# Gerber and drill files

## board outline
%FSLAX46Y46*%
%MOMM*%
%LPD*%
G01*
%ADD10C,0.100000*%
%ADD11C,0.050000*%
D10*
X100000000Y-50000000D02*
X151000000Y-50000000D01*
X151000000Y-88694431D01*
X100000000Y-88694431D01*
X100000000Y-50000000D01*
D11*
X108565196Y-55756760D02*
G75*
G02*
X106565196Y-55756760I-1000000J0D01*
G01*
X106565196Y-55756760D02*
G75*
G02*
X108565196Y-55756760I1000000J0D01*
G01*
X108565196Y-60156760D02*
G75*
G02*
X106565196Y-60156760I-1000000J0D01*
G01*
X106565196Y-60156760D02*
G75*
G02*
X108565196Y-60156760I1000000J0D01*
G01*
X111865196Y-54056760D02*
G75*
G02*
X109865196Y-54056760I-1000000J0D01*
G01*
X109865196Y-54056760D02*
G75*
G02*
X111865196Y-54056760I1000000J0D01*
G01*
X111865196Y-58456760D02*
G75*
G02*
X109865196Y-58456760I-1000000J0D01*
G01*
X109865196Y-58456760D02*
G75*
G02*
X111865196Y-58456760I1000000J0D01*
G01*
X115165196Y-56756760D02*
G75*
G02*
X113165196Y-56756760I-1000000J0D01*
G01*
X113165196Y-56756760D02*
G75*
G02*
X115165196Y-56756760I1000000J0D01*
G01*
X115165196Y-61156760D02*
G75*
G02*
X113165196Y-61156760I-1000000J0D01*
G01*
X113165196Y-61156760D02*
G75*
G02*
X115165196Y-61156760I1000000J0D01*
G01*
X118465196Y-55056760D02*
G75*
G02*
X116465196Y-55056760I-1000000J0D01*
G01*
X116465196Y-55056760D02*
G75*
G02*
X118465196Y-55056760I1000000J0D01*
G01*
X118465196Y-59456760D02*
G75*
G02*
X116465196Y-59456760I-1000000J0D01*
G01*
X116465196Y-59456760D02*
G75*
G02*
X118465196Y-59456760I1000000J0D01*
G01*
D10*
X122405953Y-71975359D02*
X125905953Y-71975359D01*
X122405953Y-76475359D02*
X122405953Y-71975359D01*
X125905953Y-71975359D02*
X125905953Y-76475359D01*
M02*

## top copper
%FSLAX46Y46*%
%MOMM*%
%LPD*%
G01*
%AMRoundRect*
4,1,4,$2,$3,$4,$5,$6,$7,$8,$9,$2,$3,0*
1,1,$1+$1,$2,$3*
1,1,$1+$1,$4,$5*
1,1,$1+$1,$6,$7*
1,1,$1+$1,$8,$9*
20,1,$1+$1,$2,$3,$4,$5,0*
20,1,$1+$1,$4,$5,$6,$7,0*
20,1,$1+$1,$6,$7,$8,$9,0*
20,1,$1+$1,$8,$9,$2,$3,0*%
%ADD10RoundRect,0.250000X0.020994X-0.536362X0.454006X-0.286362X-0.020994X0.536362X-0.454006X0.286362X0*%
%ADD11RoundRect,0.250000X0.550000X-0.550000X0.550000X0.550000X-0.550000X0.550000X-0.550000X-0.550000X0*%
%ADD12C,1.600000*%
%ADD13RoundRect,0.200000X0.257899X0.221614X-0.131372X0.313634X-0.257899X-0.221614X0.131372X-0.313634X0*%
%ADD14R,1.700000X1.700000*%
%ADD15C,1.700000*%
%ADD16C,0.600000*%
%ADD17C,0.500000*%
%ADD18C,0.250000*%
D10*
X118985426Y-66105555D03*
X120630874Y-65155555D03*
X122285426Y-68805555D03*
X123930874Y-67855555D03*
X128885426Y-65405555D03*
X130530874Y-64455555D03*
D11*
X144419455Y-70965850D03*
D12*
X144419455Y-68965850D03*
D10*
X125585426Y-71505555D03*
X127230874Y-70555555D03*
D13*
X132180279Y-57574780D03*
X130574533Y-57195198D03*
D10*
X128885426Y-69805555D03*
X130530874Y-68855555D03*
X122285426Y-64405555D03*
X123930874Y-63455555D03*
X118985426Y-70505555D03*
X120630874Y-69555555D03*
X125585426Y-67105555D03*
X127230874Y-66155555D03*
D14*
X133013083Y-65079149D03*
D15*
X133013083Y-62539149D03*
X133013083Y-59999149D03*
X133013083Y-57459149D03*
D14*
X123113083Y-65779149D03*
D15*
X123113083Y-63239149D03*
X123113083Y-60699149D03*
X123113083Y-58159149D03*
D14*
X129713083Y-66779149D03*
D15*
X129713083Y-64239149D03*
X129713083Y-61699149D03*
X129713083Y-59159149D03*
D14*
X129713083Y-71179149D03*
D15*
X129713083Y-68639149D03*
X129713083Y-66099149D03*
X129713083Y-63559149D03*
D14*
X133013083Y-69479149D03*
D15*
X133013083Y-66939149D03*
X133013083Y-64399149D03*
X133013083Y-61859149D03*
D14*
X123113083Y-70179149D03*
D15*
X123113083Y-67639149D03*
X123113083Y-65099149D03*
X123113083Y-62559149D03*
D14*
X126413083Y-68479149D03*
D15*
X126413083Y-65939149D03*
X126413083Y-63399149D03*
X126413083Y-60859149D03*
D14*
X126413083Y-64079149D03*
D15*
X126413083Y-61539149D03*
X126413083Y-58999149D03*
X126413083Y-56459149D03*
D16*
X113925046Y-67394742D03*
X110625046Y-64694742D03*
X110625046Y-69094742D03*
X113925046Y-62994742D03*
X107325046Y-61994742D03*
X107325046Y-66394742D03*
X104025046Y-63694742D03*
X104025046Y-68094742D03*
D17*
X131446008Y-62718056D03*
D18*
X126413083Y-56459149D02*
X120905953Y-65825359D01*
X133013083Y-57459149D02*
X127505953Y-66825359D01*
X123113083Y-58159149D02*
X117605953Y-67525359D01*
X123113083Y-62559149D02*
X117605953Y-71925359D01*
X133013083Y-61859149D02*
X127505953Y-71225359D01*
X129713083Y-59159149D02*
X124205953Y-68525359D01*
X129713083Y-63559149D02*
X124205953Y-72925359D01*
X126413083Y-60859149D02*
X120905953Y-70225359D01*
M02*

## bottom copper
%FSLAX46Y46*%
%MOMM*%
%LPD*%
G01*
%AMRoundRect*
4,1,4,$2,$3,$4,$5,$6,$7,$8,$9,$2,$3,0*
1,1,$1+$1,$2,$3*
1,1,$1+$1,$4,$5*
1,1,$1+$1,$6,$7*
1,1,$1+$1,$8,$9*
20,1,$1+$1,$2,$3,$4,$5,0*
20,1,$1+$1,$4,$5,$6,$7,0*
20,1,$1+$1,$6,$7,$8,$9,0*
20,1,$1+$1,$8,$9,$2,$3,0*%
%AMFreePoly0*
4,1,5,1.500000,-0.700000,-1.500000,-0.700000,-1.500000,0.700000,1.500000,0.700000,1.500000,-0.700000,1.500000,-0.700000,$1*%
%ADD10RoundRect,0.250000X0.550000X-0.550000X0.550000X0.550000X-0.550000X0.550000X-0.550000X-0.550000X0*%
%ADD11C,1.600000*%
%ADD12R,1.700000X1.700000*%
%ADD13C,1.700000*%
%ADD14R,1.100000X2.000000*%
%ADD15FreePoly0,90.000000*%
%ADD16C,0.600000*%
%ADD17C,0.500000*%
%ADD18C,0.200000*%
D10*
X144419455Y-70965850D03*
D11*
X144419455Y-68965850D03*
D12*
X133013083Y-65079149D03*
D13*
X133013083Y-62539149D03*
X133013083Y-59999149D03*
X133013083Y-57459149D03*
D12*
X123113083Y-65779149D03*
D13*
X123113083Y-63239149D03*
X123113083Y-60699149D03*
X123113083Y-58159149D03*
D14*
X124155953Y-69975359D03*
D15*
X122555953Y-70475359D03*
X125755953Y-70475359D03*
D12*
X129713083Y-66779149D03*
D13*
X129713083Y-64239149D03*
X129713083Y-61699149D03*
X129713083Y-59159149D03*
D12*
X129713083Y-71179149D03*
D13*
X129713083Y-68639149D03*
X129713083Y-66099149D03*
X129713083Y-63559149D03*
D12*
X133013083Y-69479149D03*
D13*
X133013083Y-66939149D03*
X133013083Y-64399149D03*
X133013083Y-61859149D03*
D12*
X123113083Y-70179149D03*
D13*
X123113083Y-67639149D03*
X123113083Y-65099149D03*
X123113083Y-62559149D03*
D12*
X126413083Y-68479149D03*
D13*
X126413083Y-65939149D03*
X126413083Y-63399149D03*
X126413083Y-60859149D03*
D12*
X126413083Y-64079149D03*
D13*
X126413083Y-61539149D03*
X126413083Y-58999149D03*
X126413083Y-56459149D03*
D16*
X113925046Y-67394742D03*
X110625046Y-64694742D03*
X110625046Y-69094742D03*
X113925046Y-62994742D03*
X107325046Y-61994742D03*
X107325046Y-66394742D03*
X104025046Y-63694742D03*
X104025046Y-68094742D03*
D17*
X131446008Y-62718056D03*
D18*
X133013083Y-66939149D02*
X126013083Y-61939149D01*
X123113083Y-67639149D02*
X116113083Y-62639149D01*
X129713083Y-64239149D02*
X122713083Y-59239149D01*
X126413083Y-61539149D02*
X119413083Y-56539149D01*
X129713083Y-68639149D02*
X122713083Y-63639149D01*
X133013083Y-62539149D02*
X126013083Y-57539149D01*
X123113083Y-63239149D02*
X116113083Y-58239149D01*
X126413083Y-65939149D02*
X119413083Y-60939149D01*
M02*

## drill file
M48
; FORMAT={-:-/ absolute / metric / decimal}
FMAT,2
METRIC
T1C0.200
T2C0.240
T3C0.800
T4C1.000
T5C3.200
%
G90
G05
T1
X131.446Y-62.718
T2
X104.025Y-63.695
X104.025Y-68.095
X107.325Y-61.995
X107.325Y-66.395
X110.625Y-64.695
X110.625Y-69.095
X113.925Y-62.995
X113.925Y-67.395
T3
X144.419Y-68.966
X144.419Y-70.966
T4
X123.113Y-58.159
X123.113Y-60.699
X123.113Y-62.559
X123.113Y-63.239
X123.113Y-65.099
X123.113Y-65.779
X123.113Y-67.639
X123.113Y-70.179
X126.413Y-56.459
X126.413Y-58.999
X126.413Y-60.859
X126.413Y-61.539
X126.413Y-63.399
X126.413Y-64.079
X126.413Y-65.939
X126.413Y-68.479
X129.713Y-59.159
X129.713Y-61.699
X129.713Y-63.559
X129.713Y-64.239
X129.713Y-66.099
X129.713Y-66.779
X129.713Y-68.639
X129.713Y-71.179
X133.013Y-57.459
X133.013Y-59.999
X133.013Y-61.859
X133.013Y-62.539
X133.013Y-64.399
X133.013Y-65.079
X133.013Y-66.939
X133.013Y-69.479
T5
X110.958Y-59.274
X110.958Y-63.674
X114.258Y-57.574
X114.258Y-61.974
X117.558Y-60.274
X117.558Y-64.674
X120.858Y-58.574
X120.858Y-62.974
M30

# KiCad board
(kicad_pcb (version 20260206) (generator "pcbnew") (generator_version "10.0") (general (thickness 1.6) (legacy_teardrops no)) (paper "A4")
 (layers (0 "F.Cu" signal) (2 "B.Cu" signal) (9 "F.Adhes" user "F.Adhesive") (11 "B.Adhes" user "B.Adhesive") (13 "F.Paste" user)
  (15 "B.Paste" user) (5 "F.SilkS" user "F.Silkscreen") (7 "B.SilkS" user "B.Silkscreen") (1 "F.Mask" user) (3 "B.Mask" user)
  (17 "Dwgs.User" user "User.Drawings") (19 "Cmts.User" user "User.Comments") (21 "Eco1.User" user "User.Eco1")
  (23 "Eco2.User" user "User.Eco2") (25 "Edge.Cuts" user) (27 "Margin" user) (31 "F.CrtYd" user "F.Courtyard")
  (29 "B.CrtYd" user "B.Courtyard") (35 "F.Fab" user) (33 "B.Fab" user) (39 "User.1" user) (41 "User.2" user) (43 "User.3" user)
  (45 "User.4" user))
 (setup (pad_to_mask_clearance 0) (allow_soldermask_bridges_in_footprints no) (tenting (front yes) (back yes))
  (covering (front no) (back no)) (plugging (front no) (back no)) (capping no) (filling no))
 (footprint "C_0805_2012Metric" (layer "F.Cu") (at 119.80815 65.630555 30)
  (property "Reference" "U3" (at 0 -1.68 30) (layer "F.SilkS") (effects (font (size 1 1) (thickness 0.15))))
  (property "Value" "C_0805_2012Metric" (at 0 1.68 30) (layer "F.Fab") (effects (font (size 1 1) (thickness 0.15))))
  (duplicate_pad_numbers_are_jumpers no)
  (pad "1" smd roundrect (at -0.95 0 30) (size 1 1.45) (layers "F.Cu" "F.Mask" "F.Paste") (roundrect_rratio 0.25) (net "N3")
   (clearance 0.35))
  (pad "2" smd roundrect (at 0.95 0 30) (size 1 1.45) (layers "F.Cu" "F.Mask" "F.Paste") (roundrect_rratio 0.25)))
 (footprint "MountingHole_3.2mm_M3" (layer "F.Cu") (at 117.558484 64.674067 45)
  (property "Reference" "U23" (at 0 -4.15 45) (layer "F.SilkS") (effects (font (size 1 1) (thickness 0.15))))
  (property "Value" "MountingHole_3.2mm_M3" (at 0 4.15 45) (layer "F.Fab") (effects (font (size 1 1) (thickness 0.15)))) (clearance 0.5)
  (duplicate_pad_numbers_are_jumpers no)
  (pad "" np_thru_hole circle (at 0 0 45) (size 3.2 3.2) (drill 3.2) (layers "*.Cu" "*.Mask")))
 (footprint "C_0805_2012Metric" (layer "F.Cu") (at 123.10815 68.330555 30)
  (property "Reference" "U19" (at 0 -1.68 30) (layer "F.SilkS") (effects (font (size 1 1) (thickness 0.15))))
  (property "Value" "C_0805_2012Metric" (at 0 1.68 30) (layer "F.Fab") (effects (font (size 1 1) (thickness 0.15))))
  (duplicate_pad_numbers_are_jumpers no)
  (pad "1" smd roundrect (at -0.95 0 30) (size 1 1.45) (layers "F.Cu" "F.Mask" "F.Paste") (roundrect_rratio 0.25) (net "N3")
   (clearance 0.35))
  (pad "2" smd roundrect (at 0.95 0 30) (size 1 1.45) (layers "F.Cu" "F.Mask" "F.Paste") (roundrect_rratio 0.25)))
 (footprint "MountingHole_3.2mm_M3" (layer "F.Cu") (at 114.258484 57.574067 45)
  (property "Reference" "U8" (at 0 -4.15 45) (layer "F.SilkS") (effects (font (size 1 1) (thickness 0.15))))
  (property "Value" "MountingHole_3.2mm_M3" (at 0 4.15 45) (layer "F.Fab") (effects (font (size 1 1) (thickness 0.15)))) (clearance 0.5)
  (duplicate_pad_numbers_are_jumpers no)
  (pad "" np_thru_hole circle (at 0 0 45) (size 3.2 3.2) (drill 3.2) (layers "*.Cu" "*.Mask")))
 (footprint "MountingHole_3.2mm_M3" (layer "F.Cu") (at 114.258484 61.974067 45)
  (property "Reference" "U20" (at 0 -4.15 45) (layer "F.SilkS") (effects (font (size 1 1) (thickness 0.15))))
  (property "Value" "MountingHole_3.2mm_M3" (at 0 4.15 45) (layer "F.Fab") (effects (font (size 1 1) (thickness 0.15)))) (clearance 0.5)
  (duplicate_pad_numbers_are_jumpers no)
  (pad "" np_thru_hole circle (at 0 0 45) (size 3.2 3.2) (drill 3.2) (layers "*.Cu" "*.Mask")))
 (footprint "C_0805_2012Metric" (layer "F.Cu") (at 129.70815 64.930555 30)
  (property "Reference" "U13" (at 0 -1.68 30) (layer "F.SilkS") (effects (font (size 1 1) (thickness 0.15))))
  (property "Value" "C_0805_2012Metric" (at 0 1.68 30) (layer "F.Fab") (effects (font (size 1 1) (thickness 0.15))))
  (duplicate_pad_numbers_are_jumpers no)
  (pad "1" smd roundrect (at -0.95 0 30) (size 1 1.45) (layers "F.Cu" "F.Mask" "F.Paste") (roundrect_rratio 0.25) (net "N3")
   (clearance 0.35))
  (pad "2" smd roundrect (at 0.95 0 30) (size 1 1.45) (layers "F.Cu" "F.Mask" "F.Paste") (roundrect_rratio 0.25)))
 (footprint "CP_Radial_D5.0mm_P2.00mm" (layer "F.Cu") (at 144.419455 70.96585 90)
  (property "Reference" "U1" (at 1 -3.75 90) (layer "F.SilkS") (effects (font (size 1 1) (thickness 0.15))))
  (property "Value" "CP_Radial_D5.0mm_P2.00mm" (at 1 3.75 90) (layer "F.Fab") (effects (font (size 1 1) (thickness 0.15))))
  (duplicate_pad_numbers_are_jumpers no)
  (pad "1" thru_hole roundrect (at 0 0 90) (size 1.6 1.6) (drill 0.8) (layers "*.Cu" "*.Mask") (remove_unused_layers no)
   (roundrect_rratio 0.15625) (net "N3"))
  (pad "2" thru_hole circle (at 2 0 90) (size 1.6 1.6) (drill 0.8) (layers "*.Cu" "*.Mask") (remove_unused_layers no) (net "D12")))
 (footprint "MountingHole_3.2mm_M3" (layer "F.Cu") (at 117.558484 60.274067 45)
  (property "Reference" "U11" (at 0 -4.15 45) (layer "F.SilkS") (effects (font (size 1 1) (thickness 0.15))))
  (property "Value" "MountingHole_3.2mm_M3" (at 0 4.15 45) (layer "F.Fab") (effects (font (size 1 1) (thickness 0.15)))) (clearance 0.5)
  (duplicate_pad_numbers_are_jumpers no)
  (pad "" np_thru_hole circle (at 0 0 45) (size 3.2 3.2) (drill 3.2) (layers "*.Cu" "*.Mask")))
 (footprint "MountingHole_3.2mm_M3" (layer "F.Cu") (at 110.958484 59.274067 45)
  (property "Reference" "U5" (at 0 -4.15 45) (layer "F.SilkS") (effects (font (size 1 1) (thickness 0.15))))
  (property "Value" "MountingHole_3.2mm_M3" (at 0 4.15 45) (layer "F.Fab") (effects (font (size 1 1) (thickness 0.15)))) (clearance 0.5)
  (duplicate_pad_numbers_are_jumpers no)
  (pad "" np_thru_hole circle (at 0 0 45) (size 3.2 3.2) (drill 3.2) (layers "*.Cu" "*.Mask")))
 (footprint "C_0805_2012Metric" (layer "F.Cu") (at 126.40815 71.030555 30)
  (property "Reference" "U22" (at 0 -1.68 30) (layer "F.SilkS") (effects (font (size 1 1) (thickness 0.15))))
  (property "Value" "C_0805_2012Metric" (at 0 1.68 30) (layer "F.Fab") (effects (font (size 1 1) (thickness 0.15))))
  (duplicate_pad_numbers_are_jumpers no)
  (pad "1" smd roundrect (at -0.95 0 30) (size 1 1.45) (layers "F.Cu" "F.Mask" "F.Paste") (roundrect_rratio 0.25) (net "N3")
   (clearance 0.35))
  (pad "2" smd roundrect (at 0.95 0 30) (size 1 1.45) (layers "F.Cu" "F.Mask" "F.Paste") (roundrect_rratio 0.25)))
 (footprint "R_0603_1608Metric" (layer "F.Cu") (at 131.377406 57.384989 166.7)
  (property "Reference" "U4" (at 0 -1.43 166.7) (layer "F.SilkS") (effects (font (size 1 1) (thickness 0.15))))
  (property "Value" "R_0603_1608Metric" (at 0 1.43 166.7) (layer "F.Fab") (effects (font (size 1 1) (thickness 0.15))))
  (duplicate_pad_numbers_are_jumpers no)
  (pad "1" smd roundrect (at -0.825 0 166.7) (size 0.8 0.95) (layers "F.Cu" "F.Mask" "F.Paste") (roundrect_rratio 0.25) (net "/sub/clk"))
  (pad "2" smd roundrect (at 0.825 0 166.7) (size 0.8 0.95) (layers "F.Cu" "F.Mask" "F.Paste") (roundrect_rratio 0.25) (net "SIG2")))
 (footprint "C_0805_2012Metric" (layer "F.Cu") (at 129.70815 69.330555 30)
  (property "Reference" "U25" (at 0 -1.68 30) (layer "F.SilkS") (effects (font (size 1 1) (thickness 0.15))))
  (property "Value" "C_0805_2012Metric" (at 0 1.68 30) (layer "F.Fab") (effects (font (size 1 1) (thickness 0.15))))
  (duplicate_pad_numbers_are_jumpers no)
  (pad "1" smd roundrect (at -0.95 0 30) (size 1 1.45) (layers "F.Cu" "F.Mask" "F.Paste") (roundrect_rratio 0.25) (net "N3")
   (clearance 0.35))
  (pad "2" smd roundrect (at 0.95 0 30) (size 1 1.45) (layers "F.Cu" "F.Mask" "F.Paste") (roundrect_rratio 0.25)))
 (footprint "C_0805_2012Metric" (layer "F.Cu") (at 123.10815 63.930555 30)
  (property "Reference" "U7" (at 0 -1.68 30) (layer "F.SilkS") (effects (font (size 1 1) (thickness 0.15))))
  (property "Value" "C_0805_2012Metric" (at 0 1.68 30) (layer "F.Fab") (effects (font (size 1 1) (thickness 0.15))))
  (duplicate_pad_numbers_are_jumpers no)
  (pad "1" smd roundrect (at -0.95 0 30) (size 1 1.45) (layers "F.Cu" "F.Mask" "F.Paste") (roundrect_rratio 0.25) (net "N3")
   (clearance 0.35))
  (pad "2" smd roundrect (at 0.95 0 30) (size 1 1.45) (layers "F.Cu" "F.Mask" "F.Paste") (roundrect_rratio 0.25)))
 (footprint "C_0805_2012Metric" (layer "F.Cu") (at 119.80815 70.030555 30)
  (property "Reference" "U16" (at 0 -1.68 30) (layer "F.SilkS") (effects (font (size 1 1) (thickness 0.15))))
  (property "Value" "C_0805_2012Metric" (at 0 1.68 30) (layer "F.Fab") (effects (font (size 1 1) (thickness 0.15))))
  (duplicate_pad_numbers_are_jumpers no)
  (pad "1" smd roundrect (at -0.95 0 30) (size 1 1.45) (layers "F.Cu" "F.Mask" "F.Paste") (roundrect_rratio 0.25) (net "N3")
   (clearance 0.35))
  (pad "2" smd roundrect (at 0.95 0 30) (size 1 1.45) (layers "F.Cu" "F.Mask" "F.Paste") (roundrect_rratio 0.25)))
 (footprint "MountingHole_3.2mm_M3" (layer "F.Cu") (at 110.958484 63.674067 45)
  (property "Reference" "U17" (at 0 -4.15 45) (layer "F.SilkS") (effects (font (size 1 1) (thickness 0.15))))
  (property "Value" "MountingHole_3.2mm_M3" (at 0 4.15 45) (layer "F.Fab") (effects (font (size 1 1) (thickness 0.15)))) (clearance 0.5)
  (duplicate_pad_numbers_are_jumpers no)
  (pad "" np_thru_hole circle (at 0 0 45) (size 3.2 3.2) (drill 3.2) (layers "*.Cu" "*.Mask")))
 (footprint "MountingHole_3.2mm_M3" (layer "F.Cu") (at 120.858484 58.574067 45)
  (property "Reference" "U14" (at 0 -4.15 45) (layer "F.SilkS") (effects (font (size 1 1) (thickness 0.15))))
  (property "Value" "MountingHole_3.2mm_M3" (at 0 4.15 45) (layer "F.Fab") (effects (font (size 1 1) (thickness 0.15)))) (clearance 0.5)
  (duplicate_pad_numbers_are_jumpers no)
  (pad "" np_thru_hole circle (at 0 0 45) (size 3.2 3.2) (drill 3.2) (layers "*.Cu" "*.Mask")))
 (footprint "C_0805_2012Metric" (layer "F.Cu") (at 126.40815 66.630555 30)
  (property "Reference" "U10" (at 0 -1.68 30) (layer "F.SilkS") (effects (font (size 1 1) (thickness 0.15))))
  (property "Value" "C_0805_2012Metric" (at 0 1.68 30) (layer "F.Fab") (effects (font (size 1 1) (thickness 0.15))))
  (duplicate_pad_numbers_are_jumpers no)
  (pad "1" smd roundrect (at -0.95 0 30) (size 1 1.45) (layers "F.Cu" "F.Mask" "F.Paste") (roundrect_rratio 0.25) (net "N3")
   (clearance 0.35))
  (pad "2" smd roundrect (at 0.95 0 30) (size 1 1.45) (layers "F.Cu" "F.Mask" "F.Paste") (roundrect_rratio 0.25)))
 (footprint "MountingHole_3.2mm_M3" (layer "F.Cu") (at 120.858484 62.974067 45)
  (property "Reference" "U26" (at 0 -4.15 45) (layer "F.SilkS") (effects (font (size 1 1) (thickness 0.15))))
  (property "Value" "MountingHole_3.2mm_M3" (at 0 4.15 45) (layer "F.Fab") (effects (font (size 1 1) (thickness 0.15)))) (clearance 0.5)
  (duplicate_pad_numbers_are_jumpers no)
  (pad "" np_thru_hole circle (at 0 0 45) (size 3.2 3.2) (drill 3.2) (layers "*.Cu" "*.Mask")))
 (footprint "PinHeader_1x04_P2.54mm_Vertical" (layer "B.Cu") (at 133.013083 65.079149)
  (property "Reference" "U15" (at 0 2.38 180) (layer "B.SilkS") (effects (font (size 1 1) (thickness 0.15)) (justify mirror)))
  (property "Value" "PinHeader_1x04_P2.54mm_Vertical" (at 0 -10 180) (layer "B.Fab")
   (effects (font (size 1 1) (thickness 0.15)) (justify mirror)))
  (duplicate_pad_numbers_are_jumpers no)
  (pad "1" thru_hole rect (at 0 0) (size 1.7 1.7) (drill 1) (layers "*.Cu" "*.Mask") (remove_unused_layers no) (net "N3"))
  (pad "2" thru_hole circle (at 0 -2.54) (size 1.7 1.7) (drill 1) (layers "*.Cu" "*.Mask") (remove_unused_layers no) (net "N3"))
  (pad "3" thru_hole circle (at 0 -5.08) (size 1.7 1.7) (drill 1) (layers "*.Cu" "*.Mask") (remove_unused_layers no) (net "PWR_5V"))
  (pad "4" thru_hole circle (at 0 -7.62) (size 1.7 1.7) (drill 1) (layers "*.Cu" "*.Mask") (remove_unused_layers no)))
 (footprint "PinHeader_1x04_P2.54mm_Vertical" (layer "B.Cu") (at 123.113083 65.779149)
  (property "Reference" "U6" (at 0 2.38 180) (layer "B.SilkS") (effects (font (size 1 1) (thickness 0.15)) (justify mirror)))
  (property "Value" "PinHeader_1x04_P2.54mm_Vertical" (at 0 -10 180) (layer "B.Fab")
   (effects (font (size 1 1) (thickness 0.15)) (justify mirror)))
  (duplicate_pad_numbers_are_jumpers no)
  (pad "1" thru_hole rect (at 0 0) (size 1.7 1.7) (drill 1) (layers "*.Cu" "*.Mask") (remove_unused_layers no) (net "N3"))
  (pad "2" thru_hole circle (at 0 -2.54) (size 1.7 1.7) (drill 1) (layers "*.Cu" "*.Mask") (remove_unused_layers no) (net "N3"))
  (pad "3" thru_hole circle (at 0 -5.08) (size 1.7 1.7) (drill 1) (layers "*.Cu" "*.Mask") (remove_unused_layers no) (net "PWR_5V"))
  (pad "4" thru_hole circle (at 0 -7.62) (size 1.7 1.7) (drill 1) (layers "*.Cu" "*.Mask") (remove_unused_layers no)))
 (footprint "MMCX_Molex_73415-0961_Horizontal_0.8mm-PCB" (layer "B.Cu") (at 124.155953 72.725359 90)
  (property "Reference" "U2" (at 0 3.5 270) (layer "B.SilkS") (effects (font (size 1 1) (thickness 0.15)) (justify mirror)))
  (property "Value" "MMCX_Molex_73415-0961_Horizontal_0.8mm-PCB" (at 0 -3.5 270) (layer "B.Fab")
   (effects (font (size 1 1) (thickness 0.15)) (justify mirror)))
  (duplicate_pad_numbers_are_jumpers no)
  (fp_line (start 0.75 -1.75) (end 0.75 1.75) (stroke (width 0.1) (type solid)) (layer "Edge.Cuts"))
  (fp_line (start -3.75 -1.75) (end 0.75 -1.75) (stroke (width 0.1) (type solid)) (layer "Edge.Cuts"))
  (fp_line (start 0.75 1.75) (end -3.75 1.75) (stroke (width 0.1) (type solid)) (layer "Edge.Cuts"))
  (pad "1" smd rect (at 2.75 0 90) (size 2 1.1) (layers "B.Cu" "B.Mask" "B.Paste") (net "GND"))
  (pad "2" smd custom (at 2.25 -1.6 90) (size 3 1.4) (layers "B.Cu" "B.Mask" "B.Paste") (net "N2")
   (options (clearance outline) (anchor rect)) (primitives))
  (pad "2" smd custom (at 2.25 1.6 90) (size 3 1.4) (layers "B.Cu" "B.Mask" "B.Paste") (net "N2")
   (options (clearance outline) (anchor rect)) (primitives)))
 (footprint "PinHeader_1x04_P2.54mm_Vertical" (layer "B.Cu") (at 129.713083 66.779149)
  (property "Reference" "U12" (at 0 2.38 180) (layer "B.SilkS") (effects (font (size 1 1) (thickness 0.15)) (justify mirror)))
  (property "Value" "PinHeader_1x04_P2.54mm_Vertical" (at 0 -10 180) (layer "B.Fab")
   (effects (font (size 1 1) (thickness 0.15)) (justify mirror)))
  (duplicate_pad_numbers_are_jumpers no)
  (pad "1" thru_hole rect (at 0 0) (size 1.7 1.7) (drill 1) (layers "*.Cu" "*.Mask") (remove_unused_layers no) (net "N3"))
  (pad "2" thru_hole circle (at 0 -2.54) (size 1.7 1.7) (drill 1) (layers "*.Cu" "*.Mask") (remove_unused_layers no) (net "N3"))
  (pad "3" thru_hole circle (at 0 -5.08) (size 1.7 1.7) (drill 1) (layers "*.Cu" "*.Mask") (remove_unused_layers no) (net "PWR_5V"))
  (pad "4" thru_hole circle (at 0 -7.62) (size 1.7 1.7) (drill 1) (layers "*.Cu" "*.Mask") (remove_unused_layers no)))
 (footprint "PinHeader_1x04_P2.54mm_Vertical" (layer "B.Cu") (at 129.713083 71.179149)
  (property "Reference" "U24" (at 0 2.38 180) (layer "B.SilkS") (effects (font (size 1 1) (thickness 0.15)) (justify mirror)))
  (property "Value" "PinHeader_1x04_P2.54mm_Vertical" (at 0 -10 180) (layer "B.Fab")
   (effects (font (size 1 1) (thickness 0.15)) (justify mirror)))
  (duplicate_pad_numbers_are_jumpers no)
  (pad "1" thru_hole rect (at 0 0) (size 1.7 1.7) (drill 1) (layers "*.Cu" "*.Mask") (remove_unused_layers no) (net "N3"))
  (pad "2" thru_hole circle (at 0 -2.54) (size 1.7 1.7) (drill 1) (layers "*.Cu" "*.Mask") (remove_unused_layers no) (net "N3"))
  (pad "3" thru_hole circle (at 0 -5.08) (size 1.7 1.7) (drill 1) (layers "*.Cu" "*.Mask") (remove_unused_layers no) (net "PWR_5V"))
  (pad "4" thru_hole circle (at 0 -7.62) (size 1.7 1.7) (drill 1) (layers "*.Cu" "*.Mask") (remove_unused_layers no)))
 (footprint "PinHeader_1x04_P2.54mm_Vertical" (layer "B.Cu") (at 133.013083 69.479149)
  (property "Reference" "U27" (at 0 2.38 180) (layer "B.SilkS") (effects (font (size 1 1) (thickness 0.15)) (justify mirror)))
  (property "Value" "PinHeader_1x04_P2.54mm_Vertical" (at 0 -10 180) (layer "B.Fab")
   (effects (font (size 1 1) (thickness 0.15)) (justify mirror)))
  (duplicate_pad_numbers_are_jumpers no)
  (pad "1" thru_hole rect (at 0 0) (size 1.7 1.7) (drill 1) (layers "*.Cu" "*.Mask") (remove_unused_layers no) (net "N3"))
  (pad "2" thru_hole circle (at 0 -2.54) (size 1.7 1.7) (drill 1) (layers "*.Cu" "*.Mask") (remove_unused_layers no) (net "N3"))
  (pad "3" thru_hole circle (at 0 -5.08) (size 1.7 1.7) (drill 1) (layers "*.Cu" "*.Mask") (remove_unused_layers no) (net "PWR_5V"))
  (pad "4" thru_hole circle (at 0 -7.62) (size 1.7 1.7) (drill 1) (layers "*.Cu" "*.Mask") (remove_unused_layers no)))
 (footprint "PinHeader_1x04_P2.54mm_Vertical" (layer "B.Cu") (at 123.113083 70.179149)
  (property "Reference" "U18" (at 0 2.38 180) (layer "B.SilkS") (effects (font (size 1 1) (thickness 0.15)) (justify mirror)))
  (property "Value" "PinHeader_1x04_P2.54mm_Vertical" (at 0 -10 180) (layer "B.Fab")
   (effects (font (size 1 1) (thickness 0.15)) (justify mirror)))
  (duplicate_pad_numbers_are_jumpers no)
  (pad "1" thru_hole rect (at 0 0) (size 1.7 1.7) (drill 1) (layers "*.Cu" "*.Mask") (remove_unused_layers no) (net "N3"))
  (pad "2" thru_hole circle (at 0 -2.54) (size 1.7 1.7) (drill 1) (layers "*.Cu" "*.Mask") (remove_unused_layers no) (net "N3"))
  (pad "3" thru_hole circle (at 0 -5.08) (size 1.7 1.7) (drill 1) (layers "*.Cu" "*.Mask") (remove_unused_layers no) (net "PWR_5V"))
  (pad "4" thru_hole circle (at 0 -7.62) (size 1.7 1.7) (drill 1) (layers "*.Cu" "*.Mask") (remove_unused_layers no)))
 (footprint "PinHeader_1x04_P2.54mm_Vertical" (layer "B.Cu") (at 126.413083 68.479149)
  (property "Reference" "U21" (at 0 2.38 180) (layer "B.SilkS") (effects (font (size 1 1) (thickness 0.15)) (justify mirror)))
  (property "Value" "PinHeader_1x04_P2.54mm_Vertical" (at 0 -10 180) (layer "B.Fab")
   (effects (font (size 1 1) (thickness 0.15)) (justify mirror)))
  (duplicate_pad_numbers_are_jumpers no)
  (pad "1" thru_hole rect (at 0 0) (size 1.7 1.7) (drill 1) (layers "*.Cu" "*.Mask") (remove_unused_layers no) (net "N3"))
  (pad "2" thru_hole circle (at 0 -2.54) (size 1.7 1.7) (drill 1) (layers "*.Cu" "*.Mask") (remove_unused_layers no) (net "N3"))
  (pad "3" thru_hole circle (at 0 -5.08) (size 1.7 1.7) (drill 1) (layers "*.Cu" "*.Mask") (remove_unused_layers no) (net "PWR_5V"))
  (pad "4" thru_hole circle (at 0 -7.62) (size 1.7 1.7) (drill 1) (layers "*.Cu" "*.Mask") (remove_unused_layers no)))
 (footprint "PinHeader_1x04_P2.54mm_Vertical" (layer "B.Cu") (at 126.413083 64.079149)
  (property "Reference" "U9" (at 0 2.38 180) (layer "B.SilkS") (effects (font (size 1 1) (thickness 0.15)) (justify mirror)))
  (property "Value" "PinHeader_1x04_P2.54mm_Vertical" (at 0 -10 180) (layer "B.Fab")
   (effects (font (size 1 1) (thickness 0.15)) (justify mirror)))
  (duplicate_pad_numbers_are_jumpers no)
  (pad "1" thru_hole rect (at 0 0) (size 1.7 1.7) (drill 1) (layers "*.Cu" "*.Mask") (remove_unused_layers no) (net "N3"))
  (pad "2" thru_hole circle (at 0 -2.54) (size 1.7 1.7) (drill 1) (layers "*.Cu" "*.Mask") (remove_unused_layers no) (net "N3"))
  (pad "3" thru_hole circle (at 0 -5.08) (size 1.7 1.7) (drill 1) (layers "*.Cu" "*.Mask") (remove_unused_layers no) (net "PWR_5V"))
  (pad "4" thru_hole circle (at 0 -7.62) (size 1.7 1.7) (drill 1) (layers "*.Cu" "*.Mask") (remove_unused_layers no)))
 (gr_rect (start 100 50) (end 151 88.694431) (stroke (width 0.1) (type default)) (fill no) (layer "Edge.Cuts"))
 (gr_circle (center 107.565196 55.75676) (end 108.565196 55.75676) (stroke (width 0.05) (type default)) (fill no) (layer "Edge.Cuts"))
 (gr_circle (center 107.565196 60.15676) (end 108.565196 60.15676) (stroke (width 0.05) (type default)) (fill no) (layer "Edge.Cuts"))
 (gr_circle (center 110.865196 54.05676) (end 111.865196 54.05676) (stroke (width 0.05) (type default)) (fill no) (layer "Edge.Cuts"))
 (gr_circle (center 110.865196 58.45676) (end 111.865196 58.45676) (stroke (width 0.05) (type default)) (fill no) (layer "Edge.Cuts"))
 (gr_circle (center 114.165196 56.75676) (end 115.165196 56.75676) (stroke (width 0.05) (type default)) (fill no) (layer "Edge.Cuts"))
 (gr_circle (center 114.165196 61.15676) (end 115.165196 61.15676) (stroke (width 0.05) (type default)) (fill no) (layer "Edge.Cuts"))
 (gr_circle (center 117.465196 55.05676) (end 118.465196 55.05676) (stroke (width 0.05) (type default)) (fill no) (layer "Edge.Cuts"))
 (gr_circle (center 117.465196 59.45676) (end 118.465196 59.45676) (stroke (width 0.05) (type default)) (fill no) (layer "Edge.Cuts"))
 (segment (start 126.413083 56.459149) (end 120.905953 65.825359) (width 0.25) (layer "F.Cu") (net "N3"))
 (segment (start 133.013083 57.459149) (end 127.505953 66.825359) (width 0.25) (layer "F.Cu") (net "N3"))
 (segment (start 123.113083 58.159149) (end 117.605953 67.525359) (width 0.25) (layer "F.Cu") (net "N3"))
 (segment (start 123.113083 62.559149) (end 117.605953 71.925359) (width 0.25) (layer "F.Cu") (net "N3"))
 (segment (start 133.013083 61.859149) (end 127.505953 71.225359) (width 0.25) (layer "F.Cu") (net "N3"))
 (segment (start 129.713083 59.159149) (end 124.205953 68.525359) (width 0.25) (layer "F.Cu") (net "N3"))
 (segment (start 129.713083 63.559149) (end 124.205953 72.925359) (width 0.25) (layer "F.Cu") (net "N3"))
 (segment (start 126.413083 60.859149) (end 120.905953 70.225359) (width 0.25) (layer "F.Cu") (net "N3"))
 (segment (start 133.013083 66.939149) (end 126.013083 61.939149) (width 0.2) (layer "B.Cu") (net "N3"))
 (segment (start 123.113083 67.639149) (end 116.113083 62.639149) (width 0.2) (layer "B.Cu") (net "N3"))
 (segment (start 129.713083 64.239149) (end 122.713083 59.239149) (width 0.2) (layer "B.Cu") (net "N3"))
 (segment (start 126.413083 61.539149) (end 119.413083 56.539149) (width 0.2) (layer "B.Cu") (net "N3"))
 (segment (start 129.713083 68.639149) (end 122.713083 63.639149) (width 0.2) (layer "B.Cu") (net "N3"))
 (segment (start 133.013083 62.539149) (end 126.013083 57.539149) (width 0.2) (layer "B.Cu") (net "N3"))
 (segment (start 123.113083 63.239149) (end 116.113083 58.239149) (width 0.2) (layer "B.Cu") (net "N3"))
 (segment (start 126.413083 65.939149) (end 119.413083 60.939149) (width 0.2) (layer "B.Cu") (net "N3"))
 (via (at 113.925046 67.394742) (size 0.6) (drill 0.24) (layers "F.Cu" "B.Cu") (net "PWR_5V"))
 (via (at 110.625046 64.694742) (size 0.6) (drill 0.24) (layers "F.Cu" "B.Cu") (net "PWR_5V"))
 (via (at 110.625046 69.094742) (size 0.6) (drill 0.24) (layers "F.Cu" "B.Cu") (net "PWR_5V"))
 (via (at 113.925046 62.994742) (size 0.6) (drill 0.24) (layers "F.Cu" "B.Cu") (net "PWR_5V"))
 (via (at 107.325046 61.994742) (size 0.6) (drill 0.24) (layers "F.Cu" "B.Cu") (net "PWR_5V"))
 (via (at 107.325046 66.394742) (size 0.6) (drill 0.24) (layers "F.Cu" "B.Cu") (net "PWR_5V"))
 (via (at 104.025046 63.694742) (size 0.6) (drill 0.24) (layers "F.Cu" "B.Cu") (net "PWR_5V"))
 (via (at 104.025046 68.094742) (size 0.6) (drill 0.24) (layers "F.Cu" "B.Cu") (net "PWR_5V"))
 (via (at 131.446008 62.718056) (size 0.5) (drill 0.2) (layers "F.Cu" "B.Cu") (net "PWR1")))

